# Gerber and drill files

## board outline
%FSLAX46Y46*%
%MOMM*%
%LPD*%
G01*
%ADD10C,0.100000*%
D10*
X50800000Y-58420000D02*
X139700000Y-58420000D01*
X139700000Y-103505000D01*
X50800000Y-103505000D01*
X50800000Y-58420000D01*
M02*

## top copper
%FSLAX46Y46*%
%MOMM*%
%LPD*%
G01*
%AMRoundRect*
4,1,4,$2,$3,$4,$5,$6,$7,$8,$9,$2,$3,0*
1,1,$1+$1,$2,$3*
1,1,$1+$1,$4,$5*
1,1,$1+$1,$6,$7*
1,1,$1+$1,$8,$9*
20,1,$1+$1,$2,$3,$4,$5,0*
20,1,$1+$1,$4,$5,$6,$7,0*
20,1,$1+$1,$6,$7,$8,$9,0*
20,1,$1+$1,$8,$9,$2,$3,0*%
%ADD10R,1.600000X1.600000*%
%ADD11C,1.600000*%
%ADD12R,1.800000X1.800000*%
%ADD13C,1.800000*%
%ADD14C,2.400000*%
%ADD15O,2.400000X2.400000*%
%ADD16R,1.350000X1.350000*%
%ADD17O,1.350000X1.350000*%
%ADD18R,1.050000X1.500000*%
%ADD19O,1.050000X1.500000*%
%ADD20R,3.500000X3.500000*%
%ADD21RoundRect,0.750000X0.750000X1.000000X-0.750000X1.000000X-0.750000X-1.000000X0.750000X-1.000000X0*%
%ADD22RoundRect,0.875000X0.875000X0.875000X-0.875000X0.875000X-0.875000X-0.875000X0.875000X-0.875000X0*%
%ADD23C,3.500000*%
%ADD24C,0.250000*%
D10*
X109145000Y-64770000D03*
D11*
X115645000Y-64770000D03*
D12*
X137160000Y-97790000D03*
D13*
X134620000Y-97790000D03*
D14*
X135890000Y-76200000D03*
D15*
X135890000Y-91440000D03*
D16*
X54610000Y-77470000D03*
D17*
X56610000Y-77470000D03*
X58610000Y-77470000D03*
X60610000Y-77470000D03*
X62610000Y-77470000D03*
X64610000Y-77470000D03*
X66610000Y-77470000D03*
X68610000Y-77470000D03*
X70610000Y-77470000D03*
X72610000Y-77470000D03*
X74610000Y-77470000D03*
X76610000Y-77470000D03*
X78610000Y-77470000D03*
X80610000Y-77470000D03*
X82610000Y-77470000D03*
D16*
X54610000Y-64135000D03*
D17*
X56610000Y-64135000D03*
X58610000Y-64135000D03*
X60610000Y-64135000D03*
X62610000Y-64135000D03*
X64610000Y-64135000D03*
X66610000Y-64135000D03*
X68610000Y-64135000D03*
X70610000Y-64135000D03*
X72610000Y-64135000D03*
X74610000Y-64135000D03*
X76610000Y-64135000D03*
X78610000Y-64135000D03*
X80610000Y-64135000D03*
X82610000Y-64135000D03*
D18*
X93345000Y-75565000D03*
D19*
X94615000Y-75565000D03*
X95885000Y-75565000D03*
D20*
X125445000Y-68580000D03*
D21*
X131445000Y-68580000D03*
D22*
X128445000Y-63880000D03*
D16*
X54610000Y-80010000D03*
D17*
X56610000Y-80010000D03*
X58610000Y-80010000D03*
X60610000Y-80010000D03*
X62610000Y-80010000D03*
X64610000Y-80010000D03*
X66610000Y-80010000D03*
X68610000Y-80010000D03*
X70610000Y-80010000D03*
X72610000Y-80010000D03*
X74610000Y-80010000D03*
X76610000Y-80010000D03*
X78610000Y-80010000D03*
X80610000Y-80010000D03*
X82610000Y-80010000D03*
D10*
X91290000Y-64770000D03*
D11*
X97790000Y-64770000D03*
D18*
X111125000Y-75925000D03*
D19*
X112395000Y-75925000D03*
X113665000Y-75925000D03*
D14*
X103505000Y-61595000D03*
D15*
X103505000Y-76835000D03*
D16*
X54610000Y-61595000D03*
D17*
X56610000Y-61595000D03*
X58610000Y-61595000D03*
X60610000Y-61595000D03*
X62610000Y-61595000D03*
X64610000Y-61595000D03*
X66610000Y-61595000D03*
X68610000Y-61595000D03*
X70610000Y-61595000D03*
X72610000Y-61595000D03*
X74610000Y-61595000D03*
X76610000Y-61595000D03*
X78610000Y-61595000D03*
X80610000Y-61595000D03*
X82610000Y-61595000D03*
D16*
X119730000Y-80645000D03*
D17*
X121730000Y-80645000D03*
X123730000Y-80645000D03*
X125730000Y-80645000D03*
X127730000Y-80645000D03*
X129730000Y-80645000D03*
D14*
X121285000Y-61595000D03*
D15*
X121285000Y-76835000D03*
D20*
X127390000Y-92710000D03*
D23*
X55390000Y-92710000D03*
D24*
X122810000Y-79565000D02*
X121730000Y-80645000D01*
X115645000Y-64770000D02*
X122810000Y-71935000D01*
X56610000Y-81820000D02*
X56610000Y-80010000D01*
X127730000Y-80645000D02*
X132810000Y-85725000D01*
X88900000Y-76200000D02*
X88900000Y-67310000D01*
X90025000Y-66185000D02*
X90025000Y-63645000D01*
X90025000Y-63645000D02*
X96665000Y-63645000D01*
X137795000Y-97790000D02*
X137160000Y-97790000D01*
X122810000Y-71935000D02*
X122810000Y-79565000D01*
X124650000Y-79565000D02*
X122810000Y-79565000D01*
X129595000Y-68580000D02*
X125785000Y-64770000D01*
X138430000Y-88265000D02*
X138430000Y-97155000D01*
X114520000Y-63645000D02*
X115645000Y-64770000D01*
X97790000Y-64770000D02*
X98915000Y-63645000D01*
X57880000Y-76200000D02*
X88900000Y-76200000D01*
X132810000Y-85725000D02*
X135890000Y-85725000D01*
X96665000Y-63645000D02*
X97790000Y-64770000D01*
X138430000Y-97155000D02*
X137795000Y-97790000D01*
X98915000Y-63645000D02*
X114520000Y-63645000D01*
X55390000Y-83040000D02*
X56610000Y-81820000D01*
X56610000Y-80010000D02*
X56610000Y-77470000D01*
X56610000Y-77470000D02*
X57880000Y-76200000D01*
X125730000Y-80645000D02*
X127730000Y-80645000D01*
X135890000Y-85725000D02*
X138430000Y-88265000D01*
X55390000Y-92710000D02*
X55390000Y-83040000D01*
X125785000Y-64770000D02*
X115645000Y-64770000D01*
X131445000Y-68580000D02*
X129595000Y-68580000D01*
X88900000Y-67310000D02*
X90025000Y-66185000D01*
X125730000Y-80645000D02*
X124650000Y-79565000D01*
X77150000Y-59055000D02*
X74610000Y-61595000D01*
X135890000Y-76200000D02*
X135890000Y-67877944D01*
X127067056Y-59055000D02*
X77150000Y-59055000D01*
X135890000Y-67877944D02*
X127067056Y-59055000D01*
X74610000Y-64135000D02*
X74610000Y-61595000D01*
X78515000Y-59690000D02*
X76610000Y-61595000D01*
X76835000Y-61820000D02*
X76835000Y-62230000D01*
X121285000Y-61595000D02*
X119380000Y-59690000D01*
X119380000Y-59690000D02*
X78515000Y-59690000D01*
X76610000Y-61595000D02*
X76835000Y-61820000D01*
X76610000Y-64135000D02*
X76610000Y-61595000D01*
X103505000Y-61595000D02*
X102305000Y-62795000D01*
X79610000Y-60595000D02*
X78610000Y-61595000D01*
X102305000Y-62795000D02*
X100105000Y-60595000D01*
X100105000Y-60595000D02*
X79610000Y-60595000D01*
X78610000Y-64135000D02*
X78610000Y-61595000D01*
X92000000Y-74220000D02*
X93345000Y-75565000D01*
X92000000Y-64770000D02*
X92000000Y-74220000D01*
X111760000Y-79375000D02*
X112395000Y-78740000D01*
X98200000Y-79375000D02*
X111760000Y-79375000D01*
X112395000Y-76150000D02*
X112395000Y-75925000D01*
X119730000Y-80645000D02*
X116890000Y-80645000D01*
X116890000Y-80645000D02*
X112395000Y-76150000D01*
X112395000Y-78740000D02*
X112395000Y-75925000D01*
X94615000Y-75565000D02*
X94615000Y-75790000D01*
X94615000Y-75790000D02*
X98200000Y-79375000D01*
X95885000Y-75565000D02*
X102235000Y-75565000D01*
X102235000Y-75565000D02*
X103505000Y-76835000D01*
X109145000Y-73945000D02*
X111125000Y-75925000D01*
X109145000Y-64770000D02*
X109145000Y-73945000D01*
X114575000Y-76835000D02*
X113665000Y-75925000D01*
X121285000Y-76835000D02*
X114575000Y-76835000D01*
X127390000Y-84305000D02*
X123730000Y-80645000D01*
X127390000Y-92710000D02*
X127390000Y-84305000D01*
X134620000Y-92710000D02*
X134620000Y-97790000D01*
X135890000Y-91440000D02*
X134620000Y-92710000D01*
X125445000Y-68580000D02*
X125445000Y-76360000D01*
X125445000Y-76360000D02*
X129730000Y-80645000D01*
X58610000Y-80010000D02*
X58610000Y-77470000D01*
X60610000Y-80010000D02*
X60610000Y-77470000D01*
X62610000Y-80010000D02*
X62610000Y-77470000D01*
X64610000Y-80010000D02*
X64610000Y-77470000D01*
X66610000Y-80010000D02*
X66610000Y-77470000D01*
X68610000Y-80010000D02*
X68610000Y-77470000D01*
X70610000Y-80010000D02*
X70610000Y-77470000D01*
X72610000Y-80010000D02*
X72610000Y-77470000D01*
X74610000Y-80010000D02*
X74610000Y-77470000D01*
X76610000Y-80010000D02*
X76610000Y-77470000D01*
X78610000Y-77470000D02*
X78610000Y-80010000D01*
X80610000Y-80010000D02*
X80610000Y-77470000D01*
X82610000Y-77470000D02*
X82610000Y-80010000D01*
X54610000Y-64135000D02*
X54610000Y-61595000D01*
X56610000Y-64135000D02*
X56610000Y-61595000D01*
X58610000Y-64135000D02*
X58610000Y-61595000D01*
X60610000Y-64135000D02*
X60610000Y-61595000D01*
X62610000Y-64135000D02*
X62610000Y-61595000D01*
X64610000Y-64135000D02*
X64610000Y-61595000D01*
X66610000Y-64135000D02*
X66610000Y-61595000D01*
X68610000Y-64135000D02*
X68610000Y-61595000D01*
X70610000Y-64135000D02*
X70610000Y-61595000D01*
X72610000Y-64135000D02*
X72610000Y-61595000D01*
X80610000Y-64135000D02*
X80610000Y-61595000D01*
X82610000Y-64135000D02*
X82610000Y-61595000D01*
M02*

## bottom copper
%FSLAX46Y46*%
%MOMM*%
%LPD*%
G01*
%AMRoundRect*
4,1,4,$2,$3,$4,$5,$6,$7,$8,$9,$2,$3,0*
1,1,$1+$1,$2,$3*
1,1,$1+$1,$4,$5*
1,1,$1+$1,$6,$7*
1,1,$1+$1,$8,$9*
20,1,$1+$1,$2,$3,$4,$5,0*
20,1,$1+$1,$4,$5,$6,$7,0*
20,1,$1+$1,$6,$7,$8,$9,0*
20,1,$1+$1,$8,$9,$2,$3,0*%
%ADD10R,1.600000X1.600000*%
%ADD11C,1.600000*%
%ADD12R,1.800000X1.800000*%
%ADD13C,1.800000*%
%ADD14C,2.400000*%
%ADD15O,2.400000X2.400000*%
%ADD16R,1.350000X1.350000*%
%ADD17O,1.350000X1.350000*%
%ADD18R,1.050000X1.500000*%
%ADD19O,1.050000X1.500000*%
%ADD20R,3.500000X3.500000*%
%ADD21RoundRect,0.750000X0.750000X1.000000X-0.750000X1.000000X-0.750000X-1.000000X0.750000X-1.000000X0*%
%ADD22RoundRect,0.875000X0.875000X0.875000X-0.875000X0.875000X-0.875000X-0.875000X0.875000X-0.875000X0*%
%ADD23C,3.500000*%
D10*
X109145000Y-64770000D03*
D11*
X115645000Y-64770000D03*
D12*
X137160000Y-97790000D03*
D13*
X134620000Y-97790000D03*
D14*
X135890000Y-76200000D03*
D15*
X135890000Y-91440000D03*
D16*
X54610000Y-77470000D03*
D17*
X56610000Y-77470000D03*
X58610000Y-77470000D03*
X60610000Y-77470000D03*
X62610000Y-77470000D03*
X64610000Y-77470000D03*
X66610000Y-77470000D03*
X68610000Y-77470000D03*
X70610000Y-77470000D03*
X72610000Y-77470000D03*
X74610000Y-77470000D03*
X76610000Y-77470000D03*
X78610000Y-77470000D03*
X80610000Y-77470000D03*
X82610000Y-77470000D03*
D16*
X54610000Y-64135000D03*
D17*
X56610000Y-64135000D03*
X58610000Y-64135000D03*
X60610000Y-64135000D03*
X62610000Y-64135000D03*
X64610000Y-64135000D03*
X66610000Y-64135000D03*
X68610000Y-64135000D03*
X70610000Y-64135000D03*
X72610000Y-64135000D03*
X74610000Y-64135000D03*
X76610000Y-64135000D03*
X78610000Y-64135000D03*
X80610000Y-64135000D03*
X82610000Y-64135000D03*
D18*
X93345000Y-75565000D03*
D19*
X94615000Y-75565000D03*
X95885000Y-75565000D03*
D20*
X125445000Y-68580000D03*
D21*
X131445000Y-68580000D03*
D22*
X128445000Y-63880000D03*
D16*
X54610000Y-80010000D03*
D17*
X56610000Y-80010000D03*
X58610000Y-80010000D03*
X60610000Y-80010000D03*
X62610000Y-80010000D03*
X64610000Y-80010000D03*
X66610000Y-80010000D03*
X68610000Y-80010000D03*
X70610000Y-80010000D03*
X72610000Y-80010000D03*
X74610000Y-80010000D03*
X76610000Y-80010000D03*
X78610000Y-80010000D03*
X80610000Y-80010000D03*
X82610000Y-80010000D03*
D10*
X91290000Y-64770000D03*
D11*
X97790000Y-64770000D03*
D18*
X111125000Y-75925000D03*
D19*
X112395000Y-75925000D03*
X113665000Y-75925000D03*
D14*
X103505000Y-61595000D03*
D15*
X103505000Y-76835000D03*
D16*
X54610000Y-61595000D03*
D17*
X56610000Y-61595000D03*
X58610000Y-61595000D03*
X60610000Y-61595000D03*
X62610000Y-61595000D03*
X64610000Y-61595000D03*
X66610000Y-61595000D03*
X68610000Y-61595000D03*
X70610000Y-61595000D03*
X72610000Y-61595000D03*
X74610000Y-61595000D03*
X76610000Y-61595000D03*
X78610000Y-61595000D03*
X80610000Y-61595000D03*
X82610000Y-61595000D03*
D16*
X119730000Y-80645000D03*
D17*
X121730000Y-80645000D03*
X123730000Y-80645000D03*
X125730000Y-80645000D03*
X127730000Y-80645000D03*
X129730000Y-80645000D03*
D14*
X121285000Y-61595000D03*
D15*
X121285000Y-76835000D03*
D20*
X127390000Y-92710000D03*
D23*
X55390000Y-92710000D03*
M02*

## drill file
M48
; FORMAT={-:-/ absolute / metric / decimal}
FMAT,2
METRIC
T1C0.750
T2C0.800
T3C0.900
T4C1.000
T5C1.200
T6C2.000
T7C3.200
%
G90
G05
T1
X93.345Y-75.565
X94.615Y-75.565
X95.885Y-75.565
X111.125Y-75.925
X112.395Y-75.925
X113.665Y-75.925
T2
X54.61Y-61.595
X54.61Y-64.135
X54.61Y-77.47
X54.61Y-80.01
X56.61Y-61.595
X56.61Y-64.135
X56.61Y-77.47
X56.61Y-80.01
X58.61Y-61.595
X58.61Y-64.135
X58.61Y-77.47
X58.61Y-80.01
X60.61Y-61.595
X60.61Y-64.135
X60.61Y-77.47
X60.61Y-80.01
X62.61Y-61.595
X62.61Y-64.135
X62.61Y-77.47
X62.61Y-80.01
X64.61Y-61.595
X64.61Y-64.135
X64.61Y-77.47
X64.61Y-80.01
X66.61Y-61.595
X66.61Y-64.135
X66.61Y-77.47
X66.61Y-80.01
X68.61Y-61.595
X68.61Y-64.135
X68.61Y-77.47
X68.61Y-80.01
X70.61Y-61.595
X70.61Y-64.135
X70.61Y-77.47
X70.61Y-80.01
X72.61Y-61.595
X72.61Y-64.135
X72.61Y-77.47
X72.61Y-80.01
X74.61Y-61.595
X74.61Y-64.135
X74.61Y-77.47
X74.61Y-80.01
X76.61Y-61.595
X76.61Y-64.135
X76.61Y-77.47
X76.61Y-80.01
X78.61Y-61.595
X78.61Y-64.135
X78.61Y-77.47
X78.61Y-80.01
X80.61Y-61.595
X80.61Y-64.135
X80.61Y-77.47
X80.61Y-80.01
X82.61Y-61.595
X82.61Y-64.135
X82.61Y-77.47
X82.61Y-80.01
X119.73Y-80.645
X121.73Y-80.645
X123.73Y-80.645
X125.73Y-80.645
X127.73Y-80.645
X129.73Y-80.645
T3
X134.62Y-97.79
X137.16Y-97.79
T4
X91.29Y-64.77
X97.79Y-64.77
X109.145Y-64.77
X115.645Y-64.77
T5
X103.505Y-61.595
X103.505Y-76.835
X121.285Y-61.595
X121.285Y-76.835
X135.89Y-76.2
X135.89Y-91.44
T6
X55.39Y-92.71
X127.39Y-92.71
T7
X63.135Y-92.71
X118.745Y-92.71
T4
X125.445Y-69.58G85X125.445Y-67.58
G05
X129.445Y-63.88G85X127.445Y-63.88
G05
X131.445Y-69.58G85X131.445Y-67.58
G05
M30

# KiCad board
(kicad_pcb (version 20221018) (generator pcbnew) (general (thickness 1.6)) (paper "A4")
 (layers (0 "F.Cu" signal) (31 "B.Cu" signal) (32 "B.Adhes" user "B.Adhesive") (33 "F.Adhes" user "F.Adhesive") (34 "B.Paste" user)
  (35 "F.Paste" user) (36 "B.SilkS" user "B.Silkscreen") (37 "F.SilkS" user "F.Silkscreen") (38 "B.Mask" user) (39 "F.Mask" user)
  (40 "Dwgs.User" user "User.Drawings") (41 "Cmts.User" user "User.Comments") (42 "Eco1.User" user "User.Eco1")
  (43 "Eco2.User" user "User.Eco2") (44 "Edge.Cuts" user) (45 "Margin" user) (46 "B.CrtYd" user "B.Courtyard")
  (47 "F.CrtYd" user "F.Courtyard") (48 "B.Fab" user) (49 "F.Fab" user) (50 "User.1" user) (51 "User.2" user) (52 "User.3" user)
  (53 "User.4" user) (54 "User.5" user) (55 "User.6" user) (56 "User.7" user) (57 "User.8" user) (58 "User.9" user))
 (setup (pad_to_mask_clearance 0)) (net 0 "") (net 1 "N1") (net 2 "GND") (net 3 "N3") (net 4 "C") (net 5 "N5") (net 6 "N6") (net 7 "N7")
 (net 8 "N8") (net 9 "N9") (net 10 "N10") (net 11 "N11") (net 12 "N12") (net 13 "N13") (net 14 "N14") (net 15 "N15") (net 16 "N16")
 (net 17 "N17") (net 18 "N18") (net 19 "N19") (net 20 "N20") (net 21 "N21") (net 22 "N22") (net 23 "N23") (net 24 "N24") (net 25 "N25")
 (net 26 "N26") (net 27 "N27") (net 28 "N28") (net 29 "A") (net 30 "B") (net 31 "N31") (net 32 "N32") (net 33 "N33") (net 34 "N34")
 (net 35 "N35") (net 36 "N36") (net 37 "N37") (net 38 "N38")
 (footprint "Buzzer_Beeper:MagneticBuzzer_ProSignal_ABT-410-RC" (layer "F.Cu") (at 109.145 64.77)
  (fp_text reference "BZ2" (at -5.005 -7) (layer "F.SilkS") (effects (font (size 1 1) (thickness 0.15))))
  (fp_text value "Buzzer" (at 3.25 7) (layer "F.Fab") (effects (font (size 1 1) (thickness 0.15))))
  (pad "1" thru_hole rect (at 0 0) (size 1.6 1.6) (drill 1) (layers "*.Cu" "*.Mask") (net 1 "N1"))
  (pad "2" thru_hole circle (at 6.5 0) (size 1.6 1.6) (drill 1) (layers "*.Cu" "*.Mask") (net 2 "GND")))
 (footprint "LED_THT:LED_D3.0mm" (layer "F.Cu") (at 137.16 97.79 180)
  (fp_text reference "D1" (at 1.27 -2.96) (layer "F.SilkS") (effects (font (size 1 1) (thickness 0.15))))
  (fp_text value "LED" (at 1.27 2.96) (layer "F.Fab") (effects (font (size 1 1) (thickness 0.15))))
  (pad "1" thru_hole rect (at 0 0 180) (size 1.8 1.8) (drill 0.9) (layers "*.Cu" "*.Mask") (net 2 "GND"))
  (pad "2" thru_hole circle (at 2.54 0 180) (size 1.8 1.8) (drill 0.9) (layers "*.Cu" "*.Mask") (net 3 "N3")))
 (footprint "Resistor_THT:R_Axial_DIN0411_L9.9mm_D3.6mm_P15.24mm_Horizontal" (layer "F.Cu") (at 135.89 76.2 -90)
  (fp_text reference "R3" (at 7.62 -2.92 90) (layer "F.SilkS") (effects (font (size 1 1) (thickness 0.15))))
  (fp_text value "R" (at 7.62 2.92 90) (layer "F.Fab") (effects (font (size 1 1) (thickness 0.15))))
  (pad "1" thru_hole circle (at 0 0 270) (size 2.4 2.4) (drill 1.2) (layers "*.Cu" "*.Mask") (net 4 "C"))
  (pad "2" thru_hole oval (at 15.24 0 270) (size 2.4 2.4) (drill 1.2) (layers "*.Cu" "*.Mask") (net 3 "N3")))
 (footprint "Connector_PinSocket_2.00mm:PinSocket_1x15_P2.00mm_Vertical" (layer "F.Cu") (at 54.61 77.47 90)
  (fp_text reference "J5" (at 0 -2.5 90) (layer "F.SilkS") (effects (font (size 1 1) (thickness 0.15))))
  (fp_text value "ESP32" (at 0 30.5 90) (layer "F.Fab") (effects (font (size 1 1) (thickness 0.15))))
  (pad "1" thru_hole rect (at 0 0 90) (size 1.35 1.35) (drill 0.8) (layers "*.Cu" "*.Mask") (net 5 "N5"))
  (pad "2" thru_hole oval (at 0 2 90) (size 1.35 1.35) (drill 0.8) (layers "*.Cu" "*.Mask") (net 2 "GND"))
  (pad "3" thru_hole oval (at 0 4 90) (size 1.35 1.35) (drill 0.8) (layers "*.Cu" "*.Mask") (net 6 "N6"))
  (pad "4" thru_hole oval (at 0 6 90) (size 1.35 1.35) (drill 0.8) (layers "*.Cu" "*.Mask") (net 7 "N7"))
  (pad "5" thru_hole oval (at 0 8 90) (size 1.35 1.35) (drill 0.8) (layers "*.Cu" "*.Mask") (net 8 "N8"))
  (pad "6" thru_hole oval (at 0 10 90) (size 1.35 1.35) (drill 0.8) (layers "*.Cu" "*.Mask") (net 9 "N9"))
  (pad "7" thru_hole oval (at 0 12 90) (size 1.35 1.35) (drill 0.8) (layers "*.Cu" "*.Mask") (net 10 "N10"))
  (pad "8" thru_hole oval (at 0 14 90) (size 1.35 1.35) (drill 0.8) (layers "*.Cu" "*.Mask") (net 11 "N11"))
  (pad "9" thru_hole oval (at 0 16 90) (size 1.35 1.35) (drill 0.8) (layers "*.Cu" "*.Mask") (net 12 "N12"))
  (pad "10" thru_hole oval (at 0 18 90) (size 1.35 1.35) (drill 0.8) (layers "*.Cu" "*.Mask") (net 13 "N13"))
  (pad "11" thru_hole oval (at 0 20 90) (size 1.35 1.35) (drill 0.8) (layers "*.Cu" "*.Mask") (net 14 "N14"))
  (pad "12" thru_hole oval (at 0 22 90) (size 1.35 1.35) (drill 0.8) (layers "*.Cu" "*.Mask") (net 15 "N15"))
  (pad "13" thru_hole oval (at 0 24 90) (size 1.35 1.35) (drill 0.8) (layers "*.Cu" "*.Mask") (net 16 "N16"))
  (pad "14" thru_hole oval (at 0 26 90) (size 1.35 1.35) (drill 0.8) (layers "*.Cu" "*.Mask") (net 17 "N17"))
  (pad "15" thru_hole oval (at 0 28 90) (size 1.35 1.35) (drill 0.8) (layers "*.Cu" "*.Mask") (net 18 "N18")))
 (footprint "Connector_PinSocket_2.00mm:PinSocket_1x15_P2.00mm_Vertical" (layer "F.Cu") (at 54.61 64.135 90)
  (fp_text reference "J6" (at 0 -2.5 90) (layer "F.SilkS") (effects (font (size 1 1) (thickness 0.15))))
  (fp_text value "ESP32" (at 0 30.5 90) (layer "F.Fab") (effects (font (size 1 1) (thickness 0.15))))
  (pad "1" thru_hole rect (at 0 0 90) (size 1.35 1.35) (drill 0.8) (layers "*.Cu" "*.Mask") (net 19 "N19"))
  (pad "2" thru_hole oval (at 0 2 90) (size 1.35 1.35) (drill 0.8) (layers "*.Cu" "*.Mask") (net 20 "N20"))
  (pad "3" thru_hole oval (at 0 4 90) (size 1.35 1.35) (drill 0.8) (layers "*.Cu" "*.Mask") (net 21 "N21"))
  (pad "4" thru_hole oval (at 0 6 90) (size 1.35 1.35) (drill 0.8) (layers "*.Cu" "*.Mask") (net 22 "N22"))
  (pad "5" thru_hole oval (at 0 8 90) (size 1.35 1.35) (drill 0.8) (layers "*.Cu" "*.Mask") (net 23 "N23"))
  (pad "6" thru_hole oval (at 0 10 90) (size 1.35 1.35) (drill 0.8) (layers "*.Cu" "*.Mask") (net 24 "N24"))
  (pad "7" thru_hole oval (at 0 12 90) (size 1.35 1.35) (drill 0.8) (layers "*.Cu" "*.Mask") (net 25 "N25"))
  (pad "8" thru_hole oval (at 0 14 90) (size 1.35 1.35) (drill 0.8) (layers "*.Cu" "*.Mask") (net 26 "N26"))
  (pad "9" thru_hole oval (at 0 16 90) (size 1.35 1.35) (drill 0.8) (layers "*.Cu" "*.Mask") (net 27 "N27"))
  (pad "10" thru_hole oval (at 0 18 90) (size 1.35 1.35) (drill 0.8) (layers "*.Cu" "*.Mask") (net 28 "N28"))
  (pad "11" thru_hole oval (at 0 20 90) (size 1.35 1.35) (drill 0.8) (layers "*.Cu" "*.Mask") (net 4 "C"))
  (pad "12" thru_hole oval (at 0 22 90) (size 1.35 1.35) (drill 0.8) (layers "*.Cu" "*.Mask") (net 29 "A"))
  (pad "13" thru_hole oval (at 0 24 90) (size 1.35 1.35) (drill 0.8) (layers "*.Cu" "*.Mask") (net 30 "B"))
  (pad "14" thru_hole oval (at 0 26 90) (size 1.35 1.35) (drill 0.8) (layers "*.Cu" "*.Mask") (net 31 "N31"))
  (pad "15" thru_hole oval (at 0 28 90) (size 1.35 1.35) (drill 0.8) (layers "*.Cu" "*.Mask") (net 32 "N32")))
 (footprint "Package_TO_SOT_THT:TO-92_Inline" (layer "F.Cu") (at 93.345 75.565)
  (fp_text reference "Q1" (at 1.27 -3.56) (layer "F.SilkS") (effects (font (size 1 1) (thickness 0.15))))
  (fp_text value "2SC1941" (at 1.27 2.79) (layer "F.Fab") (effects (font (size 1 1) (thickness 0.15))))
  (pad "1" thru_hole rect (at 0 0) (size 1.05 1.5) (drill 0.75) (layers "*.Cu" "*.Mask") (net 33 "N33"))
  (pad "2" thru_hole oval (at 1.27 0) (size 1.05 1.5) (drill 0.75) (layers "*.Cu" "*.Mask") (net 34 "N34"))
  (pad "3" thru_hole oval (at 2.54 0) (size 1.05 1.5) (drill 0.75) (layers "*.Cu" "*.Mask") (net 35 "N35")))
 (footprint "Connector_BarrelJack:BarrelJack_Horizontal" (layer "F.Cu") (at 125.445 68.58 180)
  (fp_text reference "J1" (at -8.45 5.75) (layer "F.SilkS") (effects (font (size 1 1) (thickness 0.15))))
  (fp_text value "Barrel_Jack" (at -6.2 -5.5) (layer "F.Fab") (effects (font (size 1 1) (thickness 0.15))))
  (pad "1" thru_hole rect (at 0 0 180) (size 3.5 3.5) (drill oval 1 3) (layers "*.Cu" "*.Mask") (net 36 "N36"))
  (pad "2" thru_hole roundrect (at -6 0 180) (size 3 3.5) (drill oval 1 3) (layers "*.Cu" "*.Mask") (roundrect_rratio 0.25) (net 2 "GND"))
  (pad "3" thru_hole roundrect (at -3 4.7 180) (size 3.5 3.5) (drill oval 3 1) (layers "*.Cu" "*.Mask") (roundrect_rratio 0.25)))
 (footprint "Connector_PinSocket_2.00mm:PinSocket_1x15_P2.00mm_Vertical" (layer "F.Cu") (at 54.61 80.01 90)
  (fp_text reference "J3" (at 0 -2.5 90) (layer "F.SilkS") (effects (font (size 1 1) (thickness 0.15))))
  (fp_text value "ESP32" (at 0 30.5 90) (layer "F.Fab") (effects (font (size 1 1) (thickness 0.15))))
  (pad "1" thru_hole rect (at 0 0 90) (size 1.35 1.35) (drill 0.8) (layers "*.Cu" "*.Mask") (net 5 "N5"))
  (pad "2" thru_hole oval (at 0 2 90) (size 1.35 1.35) (drill 0.8) (layers "*.Cu" "*.Mask") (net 2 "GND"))
  (pad "3" thru_hole oval (at 0 4 90) (size 1.35 1.35) (drill 0.8) (layers "*.Cu" "*.Mask") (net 6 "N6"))
  (pad "4" thru_hole oval (at 0 6 90) (size 1.35 1.35) (drill 0.8) (layers "*.Cu" "*.Mask") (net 7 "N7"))
  (pad "5" thru_hole oval (at 0 8 90) (size 1.35 1.35) (drill 0.8) (layers "*.Cu" "*.Mask") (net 8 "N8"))
  (pad "6" thru_hole oval (at 0 10 90) (size 1.35 1.35) (drill 0.8) (layers "*.Cu" "*.Mask") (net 9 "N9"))
  (pad "7" thru_hole oval (at 0 12 90) (size 1.35 1.35) (drill 0.8) (layers "*.Cu" "*.Mask") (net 10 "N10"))
  (pad "8" thru_hole oval (at 0 14 90) (size 1.35 1.35) (drill 0.8) (layers "*.Cu" "*.Mask") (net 11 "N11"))
  (pad "9" thru_hole oval (at 0 16 90) (size 1.35 1.35) (drill 0.8) (layers "*.Cu" "*.Mask") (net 12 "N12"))
  (pad "10" thru_hole oval (at 0 18 90) (size 1.35 1.35) (drill 0.8) (layers "*.Cu" "*.Mask") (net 13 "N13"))
  (pad "11" thru_hole oval (at 0 20 90) (size 1.35 1.35) (drill 0.8) (layers "*.Cu" "*.Mask") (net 14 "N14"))
  (pad "12" thru_hole oval (at 0 22 90) (size 1.35 1.35) (drill 0.8) (layers "*.Cu" "*.Mask") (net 15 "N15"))
  (pad "13" thru_hole oval (at 0 24 90) (size 1.35 1.35) (drill 0.8) (layers "*.Cu" "*.Mask") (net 16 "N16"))
  (pad "14" thru_hole oval (at 0 26 90) (size 1.35 1.35) (drill 0.8) (layers "*.Cu" "*.Mask") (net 17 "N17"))
  (pad "15" thru_hole oval (at 0 28 90) (size 1.35 1.35) (drill 0.8) (layers "*.Cu" "*.Mask") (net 18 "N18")))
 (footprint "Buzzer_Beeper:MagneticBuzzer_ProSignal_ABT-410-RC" (layer "F.Cu") (at 91.29 64.77)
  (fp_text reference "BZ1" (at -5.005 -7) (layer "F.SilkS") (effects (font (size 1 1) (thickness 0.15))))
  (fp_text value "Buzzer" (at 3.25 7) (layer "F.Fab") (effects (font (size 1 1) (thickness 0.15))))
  (pad "1" thru_hole rect (at 0 0) (size 1.6 1.6) (drill 1) (layers "*.Cu" "*.Mask") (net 33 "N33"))
  (pad "2" thru_hole circle (at 6.5 0) (size 1.6 1.6) (drill 1) (layers "*.Cu" "*.Mask") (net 2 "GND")))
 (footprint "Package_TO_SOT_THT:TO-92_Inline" (layer "F.Cu") (at 111.125 75.925)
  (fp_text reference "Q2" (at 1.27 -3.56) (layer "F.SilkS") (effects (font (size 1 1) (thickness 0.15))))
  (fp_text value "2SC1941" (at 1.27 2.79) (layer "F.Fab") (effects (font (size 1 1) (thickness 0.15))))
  (pad "1" thru_hole rect (at 0 0) (size 1.05 1.5) (drill 0.75) (layers "*.Cu" "*.Mask") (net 1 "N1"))
  (pad "2" thru_hole oval (at 1.27 0) (size 1.05 1.5) (drill 0.75) (layers "*.Cu" "*.Mask") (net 34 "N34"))
  (pad "3" thru_hole oval (at 2.54 0) (size 1.05 1.5) (drill 0.75) (layers "*.Cu" "*.Mask") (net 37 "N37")))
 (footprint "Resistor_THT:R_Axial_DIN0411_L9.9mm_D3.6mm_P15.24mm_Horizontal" (layer "F.Cu") (at 103.505 61.595 -90)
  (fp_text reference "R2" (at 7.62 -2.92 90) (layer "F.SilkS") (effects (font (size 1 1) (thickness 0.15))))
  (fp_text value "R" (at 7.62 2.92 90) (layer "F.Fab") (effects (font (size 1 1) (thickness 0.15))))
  (pad "1" thru_hole circle (at 0 0 270) (size 2.4 2.4) (drill 1.2) (layers "*.Cu" "*.Mask") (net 30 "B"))
  (pad "2" thru_hole oval (at 15.24 0 270) (size 2.4 2.4) (drill 1.2) (layers "*.Cu" "*.Mask") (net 35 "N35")))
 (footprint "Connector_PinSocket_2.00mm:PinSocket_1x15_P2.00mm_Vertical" (layer "F.Cu") (at 54.61 61.595 90)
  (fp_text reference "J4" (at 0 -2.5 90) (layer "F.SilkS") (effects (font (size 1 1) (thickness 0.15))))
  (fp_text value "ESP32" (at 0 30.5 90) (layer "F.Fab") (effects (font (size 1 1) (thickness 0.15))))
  (pad "1" thru_hole rect (at 0 0 90) (size 1.35 1.35) (drill 0.8) (layers "*.Cu" "*.Mask") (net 19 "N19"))
  (pad "2" thru_hole oval (at 0 2 90) (size 1.35 1.35) (drill 0.8) (layers "*.Cu" "*.Mask") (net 20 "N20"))
  (pad "3" thru_hole oval (at 0 4 90) (size 1.35 1.35) (drill 0.8) (layers "*.Cu" "*.Mask") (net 21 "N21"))
  (pad "4" thru_hole oval (at 0 6 90) (size 1.35 1.35) (drill 0.8) (layers "*.Cu" "*.Mask") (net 22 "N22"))
  (pad "5" thru_hole oval (at 0 8 90) (size 1.35 1.35) (drill 0.8) (layers "*.Cu" "*.Mask") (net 23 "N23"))
  (pad "6" thru_hole oval (at 0 10 90) (size 1.35 1.35) (drill 0.8) (layers "*.Cu" "*.Mask") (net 24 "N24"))
  (pad "7" thru_hole oval (at 0 12 90) (size 1.35 1.35) (drill 0.8) (layers "*.Cu" "*.Mask") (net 25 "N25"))
  (pad "8" thru_hole oval (at 0 14 90) (size 1.35 1.35) (drill 0.8) (layers "*.Cu" "*.Mask") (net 26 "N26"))
  (pad "9" thru_hole oval (at 0 16 90) (size 1.35 1.35) (drill 0.8) (layers "*.Cu" "*.Mask") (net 27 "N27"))
  (pad "10" thru_hole oval (at 0 18 90) (size 1.35 1.35) (drill 0.8) (layers "*.Cu" "*.Mask") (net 28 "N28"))
  (pad "11" thru_hole oval (at 0 20 90) (size 1.35 1.35) (drill 0.8) (layers "*.Cu" "*.Mask") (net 4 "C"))
  (pad "12" thru_hole oval (at 0 22 90) (size 1.35 1.35) (drill 0.8) (layers "*.Cu" "*.Mask") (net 29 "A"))
  (pad "13" thru_hole oval (at 0 24 90) (size 1.35 1.35) (drill 0.8) (layers "*.Cu" "*.Mask") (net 30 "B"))
  (pad "14" thru_hole oval (at 0 26 90) (size 1.35 1.35) (drill 0.8) (layers "*.Cu" "*.Mask") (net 31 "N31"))
  (pad "15" thru_hole oval (at 0 28 90) (size 1.35 1.35) (drill 0.8) (layers "*.Cu" "*.Mask") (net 32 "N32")))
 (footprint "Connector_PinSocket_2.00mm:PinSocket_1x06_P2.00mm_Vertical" (layer "F.Cu") (at 119.73 80.645 90)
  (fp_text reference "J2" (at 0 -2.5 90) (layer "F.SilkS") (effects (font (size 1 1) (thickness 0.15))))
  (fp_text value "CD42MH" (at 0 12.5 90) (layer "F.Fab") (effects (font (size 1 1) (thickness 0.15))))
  (pad "1" thru_hole rect (at 0 0 90) (size 1.35 1.35) (drill 0.8) (layers "*.Cu" "*.Mask") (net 34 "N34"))
  (pad "2" thru_hole oval (at 0 2 90) (size 1.35 1.35) (drill 0.8) (layers "*.Cu" "*.Mask") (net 2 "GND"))
  (pad "3" thru_hole oval (at 0 4 90) (size 1.35 1.35) (drill 0.8) (layers "*.Cu" "*.Mask") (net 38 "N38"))
  (pad "4" thru_hole oval (at 0 6 90) (size 1.35 1.35) (drill 0.8) (layers "*.Cu" "*.Mask") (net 2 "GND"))
  (pad "5" thru_hole oval (at 0 8 90) (size 1.35 1.35) (drill 0.8) (layers "*.Cu" "*.Mask") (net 2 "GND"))
  (pad "6" thru_hole oval (at 0 10 90) (size 1.35 1.35) (drill 0.8) (layers "*.Cu" "*.Mask") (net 36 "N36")))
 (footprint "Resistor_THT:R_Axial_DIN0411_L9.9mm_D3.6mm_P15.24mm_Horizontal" (layer "F.Cu") (at 121.285 61.595 -90)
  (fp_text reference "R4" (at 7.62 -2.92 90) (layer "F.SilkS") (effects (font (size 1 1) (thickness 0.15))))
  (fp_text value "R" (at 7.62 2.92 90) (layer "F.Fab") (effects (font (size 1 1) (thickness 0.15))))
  (pad "1" thru_hole circle (at 0 0 270) (size 2.4 2.4) (drill 1.2) (layers "*.Cu" "*.Mask") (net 29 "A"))
  (pad "2" thru_hole oval (at 15.24 0 270) (size 2.4 2.4) (drill 1.2) (layers "*.Cu" "*.Mask") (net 37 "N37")))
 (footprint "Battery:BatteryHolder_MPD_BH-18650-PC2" (layer "B.Cu") (at 127.39 92.71 180)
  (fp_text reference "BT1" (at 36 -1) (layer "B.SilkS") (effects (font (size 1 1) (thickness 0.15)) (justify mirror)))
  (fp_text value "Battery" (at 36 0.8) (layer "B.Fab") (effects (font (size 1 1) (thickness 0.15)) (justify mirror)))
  (pad "" np_thru_hole circle (at 8.645 0 180) (size 3.2 3.2) (drill 3.2) (layers "*.Cu" "*.Mask"))
  (pad "" np_thru_hole circle (at 64.255 0 180) (size 3.2 3.2) (drill 3.2) (layers "*.Cu" "*.Mask"))
  (pad "1" thru_hole rect (at 0 0 180) (size 3.5 3.5) (drill 2) (layers "*.Cu" "*.Mask") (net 38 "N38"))
  (pad "2" thru_hole circle (at 72 0 180) (size 3.5 3.5) (drill 2) (layers "*.Cu" "*.Mask") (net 2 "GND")))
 (gr_rect (start 50.8 58.42) (end 139.7 103.505) (stroke (width 0.1) (type default)) (fill none) (layer "Edge.Cuts"))
 (segment (start 122.81 79.565) (end 121.73 80.645) (width 0.25) (layer "F.Cu") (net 2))
 (segment (start 115.645 64.77) (end 122.81 71.935) (width 0.25) (layer "F.Cu") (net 2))
 (segment (start 56.61 81.82) (end 56.61 80.01) (width 0.25) (layer "F.Cu") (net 2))
 (segment (start 127.73 80.645) (end 132.81 85.725) (width 0.25) (layer "F.Cu") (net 2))
 (segment (start 88.9 76.2) (end 88.9 67.31) (width 0.25) (layer "F.Cu") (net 2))
 (segment (start 90.025 66.185) (end 90.025 63.645) (width 0.25) (layer "F.Cu") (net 2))
 (segment (start 90.025 63.645) (end 96.665 63.645) (width 0.25) (layer "F.Cu") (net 2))
 (segment (start 137.795 97.79) (end 137.16 97.79) (width 0.25) (layer "F.Cu") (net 2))
 (segment (start 122.81 71.935) (end 122.81 79.565) (width 0.25) (layer "F.Cu") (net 2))
 (segment (start 124.65 79.565) (end 122.81 79.565) (width 0.25) (layer "F.Cu") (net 2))
 (segment (start 129.595 68.58) (end 125.785 64.77) (width 0.25) (layer "F.Cu") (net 2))
 (segment (start 138.43 88.265) (end 138.43 97.155) (width 0.25) (layer "F.Cu") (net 2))
 (segment (start 114.52 63.645) (end 115.645 64.77) (width 0.25) (layer "F.Cu") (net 2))
 (segment (start 97.79 64.77) (end 98.915 63.645) (width 0.25) (layer "F.Cu") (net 2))
 (segment (start 57.88 76.2) (end 88.9 76.2) (width 0.25) (layer "F.Cu") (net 2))
 (segment (start 132.81 85.725) (end 135.89 85.725) (width 0.25) (layer "F.Cu") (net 2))
 (segment (start 96.665 63.645) (end 97.79 64.77) (width 0.25) (layer "F.Cu") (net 2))
 (segment (start 138.43 97.155) (end 137.795 97.79) (width 0.25) (layer "F.Cu") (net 2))
 (segment (start 98.915 63.645) (end 114.52 63.645) (width 0.25) (layer "F.Cu") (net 2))
 (segment (start 55.39 83.04) (end 56.61 81.82) (width 0.25) (layer "F.Cu") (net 2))
 (segment (start 56.61 80.01) (end 56.61 77.47) (width 0.25) (layer "F.Cu") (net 2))
 (segment (start 56.61 77.47) (end 57.88 76.2) (width 0.25) (layer "F.Cu") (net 2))
 (segment (start 125.73 80.645) (end 127.73 80.645) (width 0.25) (layer "F.Cu") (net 2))
 (segment (start 135.89 85.725) (end 138.43 88.265) (width 0.25) (layer "F.Cu") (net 2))
 (segment (start 55.39 92.71) (end 55.39 83.04) (width 0.25) (layer "F.Cu") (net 2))
 (segment (start 125.785 64.77) (end 115.645 64.77) (width 0.25) (layer "F.Cu") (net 2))
 (segment (start 131.445 68.58) (end 129.595 68.58) (width 0.25) (layer "F.Cu") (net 2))
 (segment (start 88.9 67.31) (end 90.025 66.185) (width 0.25) (layer "F.Cu") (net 2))
 (segment (start 125.73 80.645) (end 124.65 79.565) (width 0.25) (layer "F.Cu") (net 2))
 (segment (start 77.15 59.055) (end 74.61 61.595) (width 0.25) (layer "F.Cu") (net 4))
 (segment (start 135.89 76.2) (end 135.89 67.877944) (width 0.25) (layer "F.Cu") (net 4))
 (segment (start 127.067056 59.055) (end 77.15 59.055) (width 0.25) (layer "F.Cu") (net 4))
 (segment (start 135.89 67.877944) (end 127.067056 59.055) (width 0.25) (layer "F.Cu") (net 4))
 (segment (start 74.61 64.135) (end 74.61 61.595) (width 0.25) (layer "F.Cu") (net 4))
 (segment (start 78.515 59.69) (end 76.61 61.595) (width 0.25) (layer "F.Cu") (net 29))
 (segment (start 76.835 61.82) (end 76.835 62.23) (width 0.25) (layer "F.Cu") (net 29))
 (segment (start 121.285 61.595) (end 119.38 59.69) (width 0.25) (layer "F.Cu") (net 29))
 (segment (start 119.38 59.69) (end 78.515 59.69) (width 0.25) (layer "F.Cu") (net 29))
 (segment (start 76.61 61.595) (end 76.835 61.82) (width 0.25) (layer "F.Cu") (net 29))
 (segment (start 76.61 64.135) (end 76.61 61.595) (width 0.25) (layer "F.Cu") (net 29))
 (segment (start 103.505 61.595) (end 102.305 62.795) (width 0.25) (layer "F.Cu") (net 30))
 (segment (start 79.61 60.595) (end 78.61 61.595) (width 0.25) (layer "F.Cu") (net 30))
 (segment (start 102.305 62.795) (end 100.105 60.595) (width 0.25) (layer "F.Cu") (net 30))
 (segment (start 100.105 60.595) (end 79.61 60.595) (width 0.25) (layer "F.Cu") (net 30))
 (segment (start 78.61 64.135) (end 78.61 61.595) (width 0.25) (layer "F.Cu") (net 30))
 (segment (start 92 74.22) (end 93.345 75.565) (width 0.25) (layer "F.Cu") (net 33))
 (segment (start 92 64.77) (end 92 74.22) (width 0.25) (layer "F.Cu") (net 33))
 (segment (start 111.76 79.375) (end 112.395 78.74) (width 0.25) (layer "F.Cu") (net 34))
 (segment (start 98.2 79.375) (end 111.76 79.375) (width 0.25) (layer "F.Cu") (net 34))
 (segment (start 112.395 76.15) (end 112.395 75.925) (width 0.25) (layer "F.Cu") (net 34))
 (segment (start 119.73 80.645) (end 116.89 80.645) (width 0.25) (layer "F.Cu") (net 34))
 (segment (start 116.89 80.645) (end 112.395 76.15) (width 0.25) (layer "F.Cu") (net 34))
 (segment (start 112.395 78.74) (end 112.395 75.925) (width 0.25) (layer "F.Cu") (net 34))
 (segment (start 94.615 75.565) (end 94.615 75.79) (width 0.25) (layer "F.Cu") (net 34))
 (segment (start 94.615 75.79) (end 98.2 79.375) (width 0.25) (layer "F.Cu") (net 34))
 (segment (start 95.885 75.565) (end 102.235 75.565) (width 0.25) (layer "F.Cu") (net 35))
 (segment (start 102.235 75.565) (end 103.505 76.835) (width 0.25) (layer "F.Cu") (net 35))
 (segment (start 109.145 73.945) (end 111.125 75.925) (width 0.25) (layer "F.Cu") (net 1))
 (segment (start 109.145 64.77) (end 109.145 73.945) (width 0.25) (layer "F.Cu") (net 1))
 (segment (start 114.575 76.835) (end 113.665 75.925) (width 0.25) (layer "F.Cu") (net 37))
 (segment (start 121.285 76.835) (end 114.575 76.835) (width 0.25) (layer "F.Cu") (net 37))
 (segment (start 127.39 84.305) (end 123.73 80.645) (width 0.25) (layer "F.Cu") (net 38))
 (segment (start 127.39 92.71) (end 127.39 84.305) (width 0.25) (layer "F.Cu") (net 38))
 (segment (start 134.62 92.71) (end 134.62 97.79) (width 0.25) (layer "F.Cu") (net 3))
 (segment (start 135.89 91.44) (end 134.62 92.71) (width 0.25) (layer "F.Cu") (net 3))
 (segment (start 125.445 68.58) (end 125.445 76.36) (width 0.25) (layer "F.Cu") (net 36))
 (segment (start 125.445 76.36) (end 129.73 80.645) (width 0.25) (layer "F.Cu") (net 36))
 (segment (start 58.61 80.01) (end 58.61 77.47) (width 0.25) (layer "F.Cu") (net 6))
 (segment (start 60.61 80.01) (end 60.61 77.47) (width 0.25) (layer "F.Cu") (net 7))
 (segment (start 62.61 80.01) (end 62.61 77.47) (width 0.25) (layer "F.Cu") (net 8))
 (segment (start 64.61 80.01) (end 64.61 77.47) (width 0.25) (layer "F.Cu") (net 9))
 (segment (start 66.61 80.01) (end 66.61 77.47) (width 0.25) (layer "F.Cu") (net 10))
 (segment (start 68.61 80.01) (end 68.61 77.47) (width 0.25) (layer "F.Cu") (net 11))
 (segment (start 70.61 80.01) (end 70.61 77.47) (width 0.25) (layer "F.Cu") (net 12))
 (segment (start 72.61 80.01) (end 72.61 77.47) (width 0.25) (layer "F.Cu") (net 13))
 (segment (start 74.61 80.01) (end 74.61 77.47) (width 0.25) (layer "F.Cu") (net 14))
 (segment (start 76.61 80.01) (end 76.61 77.47) (width 0.25) (layer "F.Cu") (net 15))
 (segment (start 78.61 77.47) (end 78.61 80.01) (width 0.25) (layer "F.Cu") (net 16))
 (segment (start 80.61 80.01) (end 80.61 77.47) (width 0.25) (layer "F.Cu") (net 17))
 (segment (start 82.61 77.47) (end 82.61 80.01) (width 0.25) (layer "F.Cu") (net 18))
 (segment (start 54.61 64.135) (end 54.61 61.595) (width 0.25) (layer "F.Cu") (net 19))
 (segment (start 56.61 64.135) (end 56.61 61.595) (width 0.25) (layer "F.Cu") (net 20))
 (segment (start 58.61 64.135) (end 58.61 61.595) (width 0.25) (layer "F.Cu") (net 21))
 (segment (start 60.61 64.135) (end 60.61 61.595) (width 0.25) (layer "F.Cu") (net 22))
 (segment (start 62.61 64.135) (end 62.61 61.595) (width 0.25) (layer "F.Cu") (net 23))
 (segment (start 64.61 64.135) (end 64.61 61.595) (width 0.25) (layer "F.Cu") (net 24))
 (segment (start 66.61 64.135) (end 66.61 61.595) (width 0.25) (layer "F.Cu") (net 25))
 (segment (start 68.61 64.135) (end 68.61 61.595) (width 0.25) (layer "F.Cu") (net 26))
 (segment (start 70.61 64.135) (end 70.61 61.595) (width 0.25) (layer "F.Cu") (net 27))
 (segment (start 72.61 64.135) (end 72.61 61.595) (width 0.25) (layer "F.Cu") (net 28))
 (segment (start 80.61 64.135) (end 80.61 61.595) (width 0.25) (layer "F.Cu") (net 31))
 (segment (start 82.61 64.135) (end 82.61 61.595) (width 0.25) (layer "F.Cu") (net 32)))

